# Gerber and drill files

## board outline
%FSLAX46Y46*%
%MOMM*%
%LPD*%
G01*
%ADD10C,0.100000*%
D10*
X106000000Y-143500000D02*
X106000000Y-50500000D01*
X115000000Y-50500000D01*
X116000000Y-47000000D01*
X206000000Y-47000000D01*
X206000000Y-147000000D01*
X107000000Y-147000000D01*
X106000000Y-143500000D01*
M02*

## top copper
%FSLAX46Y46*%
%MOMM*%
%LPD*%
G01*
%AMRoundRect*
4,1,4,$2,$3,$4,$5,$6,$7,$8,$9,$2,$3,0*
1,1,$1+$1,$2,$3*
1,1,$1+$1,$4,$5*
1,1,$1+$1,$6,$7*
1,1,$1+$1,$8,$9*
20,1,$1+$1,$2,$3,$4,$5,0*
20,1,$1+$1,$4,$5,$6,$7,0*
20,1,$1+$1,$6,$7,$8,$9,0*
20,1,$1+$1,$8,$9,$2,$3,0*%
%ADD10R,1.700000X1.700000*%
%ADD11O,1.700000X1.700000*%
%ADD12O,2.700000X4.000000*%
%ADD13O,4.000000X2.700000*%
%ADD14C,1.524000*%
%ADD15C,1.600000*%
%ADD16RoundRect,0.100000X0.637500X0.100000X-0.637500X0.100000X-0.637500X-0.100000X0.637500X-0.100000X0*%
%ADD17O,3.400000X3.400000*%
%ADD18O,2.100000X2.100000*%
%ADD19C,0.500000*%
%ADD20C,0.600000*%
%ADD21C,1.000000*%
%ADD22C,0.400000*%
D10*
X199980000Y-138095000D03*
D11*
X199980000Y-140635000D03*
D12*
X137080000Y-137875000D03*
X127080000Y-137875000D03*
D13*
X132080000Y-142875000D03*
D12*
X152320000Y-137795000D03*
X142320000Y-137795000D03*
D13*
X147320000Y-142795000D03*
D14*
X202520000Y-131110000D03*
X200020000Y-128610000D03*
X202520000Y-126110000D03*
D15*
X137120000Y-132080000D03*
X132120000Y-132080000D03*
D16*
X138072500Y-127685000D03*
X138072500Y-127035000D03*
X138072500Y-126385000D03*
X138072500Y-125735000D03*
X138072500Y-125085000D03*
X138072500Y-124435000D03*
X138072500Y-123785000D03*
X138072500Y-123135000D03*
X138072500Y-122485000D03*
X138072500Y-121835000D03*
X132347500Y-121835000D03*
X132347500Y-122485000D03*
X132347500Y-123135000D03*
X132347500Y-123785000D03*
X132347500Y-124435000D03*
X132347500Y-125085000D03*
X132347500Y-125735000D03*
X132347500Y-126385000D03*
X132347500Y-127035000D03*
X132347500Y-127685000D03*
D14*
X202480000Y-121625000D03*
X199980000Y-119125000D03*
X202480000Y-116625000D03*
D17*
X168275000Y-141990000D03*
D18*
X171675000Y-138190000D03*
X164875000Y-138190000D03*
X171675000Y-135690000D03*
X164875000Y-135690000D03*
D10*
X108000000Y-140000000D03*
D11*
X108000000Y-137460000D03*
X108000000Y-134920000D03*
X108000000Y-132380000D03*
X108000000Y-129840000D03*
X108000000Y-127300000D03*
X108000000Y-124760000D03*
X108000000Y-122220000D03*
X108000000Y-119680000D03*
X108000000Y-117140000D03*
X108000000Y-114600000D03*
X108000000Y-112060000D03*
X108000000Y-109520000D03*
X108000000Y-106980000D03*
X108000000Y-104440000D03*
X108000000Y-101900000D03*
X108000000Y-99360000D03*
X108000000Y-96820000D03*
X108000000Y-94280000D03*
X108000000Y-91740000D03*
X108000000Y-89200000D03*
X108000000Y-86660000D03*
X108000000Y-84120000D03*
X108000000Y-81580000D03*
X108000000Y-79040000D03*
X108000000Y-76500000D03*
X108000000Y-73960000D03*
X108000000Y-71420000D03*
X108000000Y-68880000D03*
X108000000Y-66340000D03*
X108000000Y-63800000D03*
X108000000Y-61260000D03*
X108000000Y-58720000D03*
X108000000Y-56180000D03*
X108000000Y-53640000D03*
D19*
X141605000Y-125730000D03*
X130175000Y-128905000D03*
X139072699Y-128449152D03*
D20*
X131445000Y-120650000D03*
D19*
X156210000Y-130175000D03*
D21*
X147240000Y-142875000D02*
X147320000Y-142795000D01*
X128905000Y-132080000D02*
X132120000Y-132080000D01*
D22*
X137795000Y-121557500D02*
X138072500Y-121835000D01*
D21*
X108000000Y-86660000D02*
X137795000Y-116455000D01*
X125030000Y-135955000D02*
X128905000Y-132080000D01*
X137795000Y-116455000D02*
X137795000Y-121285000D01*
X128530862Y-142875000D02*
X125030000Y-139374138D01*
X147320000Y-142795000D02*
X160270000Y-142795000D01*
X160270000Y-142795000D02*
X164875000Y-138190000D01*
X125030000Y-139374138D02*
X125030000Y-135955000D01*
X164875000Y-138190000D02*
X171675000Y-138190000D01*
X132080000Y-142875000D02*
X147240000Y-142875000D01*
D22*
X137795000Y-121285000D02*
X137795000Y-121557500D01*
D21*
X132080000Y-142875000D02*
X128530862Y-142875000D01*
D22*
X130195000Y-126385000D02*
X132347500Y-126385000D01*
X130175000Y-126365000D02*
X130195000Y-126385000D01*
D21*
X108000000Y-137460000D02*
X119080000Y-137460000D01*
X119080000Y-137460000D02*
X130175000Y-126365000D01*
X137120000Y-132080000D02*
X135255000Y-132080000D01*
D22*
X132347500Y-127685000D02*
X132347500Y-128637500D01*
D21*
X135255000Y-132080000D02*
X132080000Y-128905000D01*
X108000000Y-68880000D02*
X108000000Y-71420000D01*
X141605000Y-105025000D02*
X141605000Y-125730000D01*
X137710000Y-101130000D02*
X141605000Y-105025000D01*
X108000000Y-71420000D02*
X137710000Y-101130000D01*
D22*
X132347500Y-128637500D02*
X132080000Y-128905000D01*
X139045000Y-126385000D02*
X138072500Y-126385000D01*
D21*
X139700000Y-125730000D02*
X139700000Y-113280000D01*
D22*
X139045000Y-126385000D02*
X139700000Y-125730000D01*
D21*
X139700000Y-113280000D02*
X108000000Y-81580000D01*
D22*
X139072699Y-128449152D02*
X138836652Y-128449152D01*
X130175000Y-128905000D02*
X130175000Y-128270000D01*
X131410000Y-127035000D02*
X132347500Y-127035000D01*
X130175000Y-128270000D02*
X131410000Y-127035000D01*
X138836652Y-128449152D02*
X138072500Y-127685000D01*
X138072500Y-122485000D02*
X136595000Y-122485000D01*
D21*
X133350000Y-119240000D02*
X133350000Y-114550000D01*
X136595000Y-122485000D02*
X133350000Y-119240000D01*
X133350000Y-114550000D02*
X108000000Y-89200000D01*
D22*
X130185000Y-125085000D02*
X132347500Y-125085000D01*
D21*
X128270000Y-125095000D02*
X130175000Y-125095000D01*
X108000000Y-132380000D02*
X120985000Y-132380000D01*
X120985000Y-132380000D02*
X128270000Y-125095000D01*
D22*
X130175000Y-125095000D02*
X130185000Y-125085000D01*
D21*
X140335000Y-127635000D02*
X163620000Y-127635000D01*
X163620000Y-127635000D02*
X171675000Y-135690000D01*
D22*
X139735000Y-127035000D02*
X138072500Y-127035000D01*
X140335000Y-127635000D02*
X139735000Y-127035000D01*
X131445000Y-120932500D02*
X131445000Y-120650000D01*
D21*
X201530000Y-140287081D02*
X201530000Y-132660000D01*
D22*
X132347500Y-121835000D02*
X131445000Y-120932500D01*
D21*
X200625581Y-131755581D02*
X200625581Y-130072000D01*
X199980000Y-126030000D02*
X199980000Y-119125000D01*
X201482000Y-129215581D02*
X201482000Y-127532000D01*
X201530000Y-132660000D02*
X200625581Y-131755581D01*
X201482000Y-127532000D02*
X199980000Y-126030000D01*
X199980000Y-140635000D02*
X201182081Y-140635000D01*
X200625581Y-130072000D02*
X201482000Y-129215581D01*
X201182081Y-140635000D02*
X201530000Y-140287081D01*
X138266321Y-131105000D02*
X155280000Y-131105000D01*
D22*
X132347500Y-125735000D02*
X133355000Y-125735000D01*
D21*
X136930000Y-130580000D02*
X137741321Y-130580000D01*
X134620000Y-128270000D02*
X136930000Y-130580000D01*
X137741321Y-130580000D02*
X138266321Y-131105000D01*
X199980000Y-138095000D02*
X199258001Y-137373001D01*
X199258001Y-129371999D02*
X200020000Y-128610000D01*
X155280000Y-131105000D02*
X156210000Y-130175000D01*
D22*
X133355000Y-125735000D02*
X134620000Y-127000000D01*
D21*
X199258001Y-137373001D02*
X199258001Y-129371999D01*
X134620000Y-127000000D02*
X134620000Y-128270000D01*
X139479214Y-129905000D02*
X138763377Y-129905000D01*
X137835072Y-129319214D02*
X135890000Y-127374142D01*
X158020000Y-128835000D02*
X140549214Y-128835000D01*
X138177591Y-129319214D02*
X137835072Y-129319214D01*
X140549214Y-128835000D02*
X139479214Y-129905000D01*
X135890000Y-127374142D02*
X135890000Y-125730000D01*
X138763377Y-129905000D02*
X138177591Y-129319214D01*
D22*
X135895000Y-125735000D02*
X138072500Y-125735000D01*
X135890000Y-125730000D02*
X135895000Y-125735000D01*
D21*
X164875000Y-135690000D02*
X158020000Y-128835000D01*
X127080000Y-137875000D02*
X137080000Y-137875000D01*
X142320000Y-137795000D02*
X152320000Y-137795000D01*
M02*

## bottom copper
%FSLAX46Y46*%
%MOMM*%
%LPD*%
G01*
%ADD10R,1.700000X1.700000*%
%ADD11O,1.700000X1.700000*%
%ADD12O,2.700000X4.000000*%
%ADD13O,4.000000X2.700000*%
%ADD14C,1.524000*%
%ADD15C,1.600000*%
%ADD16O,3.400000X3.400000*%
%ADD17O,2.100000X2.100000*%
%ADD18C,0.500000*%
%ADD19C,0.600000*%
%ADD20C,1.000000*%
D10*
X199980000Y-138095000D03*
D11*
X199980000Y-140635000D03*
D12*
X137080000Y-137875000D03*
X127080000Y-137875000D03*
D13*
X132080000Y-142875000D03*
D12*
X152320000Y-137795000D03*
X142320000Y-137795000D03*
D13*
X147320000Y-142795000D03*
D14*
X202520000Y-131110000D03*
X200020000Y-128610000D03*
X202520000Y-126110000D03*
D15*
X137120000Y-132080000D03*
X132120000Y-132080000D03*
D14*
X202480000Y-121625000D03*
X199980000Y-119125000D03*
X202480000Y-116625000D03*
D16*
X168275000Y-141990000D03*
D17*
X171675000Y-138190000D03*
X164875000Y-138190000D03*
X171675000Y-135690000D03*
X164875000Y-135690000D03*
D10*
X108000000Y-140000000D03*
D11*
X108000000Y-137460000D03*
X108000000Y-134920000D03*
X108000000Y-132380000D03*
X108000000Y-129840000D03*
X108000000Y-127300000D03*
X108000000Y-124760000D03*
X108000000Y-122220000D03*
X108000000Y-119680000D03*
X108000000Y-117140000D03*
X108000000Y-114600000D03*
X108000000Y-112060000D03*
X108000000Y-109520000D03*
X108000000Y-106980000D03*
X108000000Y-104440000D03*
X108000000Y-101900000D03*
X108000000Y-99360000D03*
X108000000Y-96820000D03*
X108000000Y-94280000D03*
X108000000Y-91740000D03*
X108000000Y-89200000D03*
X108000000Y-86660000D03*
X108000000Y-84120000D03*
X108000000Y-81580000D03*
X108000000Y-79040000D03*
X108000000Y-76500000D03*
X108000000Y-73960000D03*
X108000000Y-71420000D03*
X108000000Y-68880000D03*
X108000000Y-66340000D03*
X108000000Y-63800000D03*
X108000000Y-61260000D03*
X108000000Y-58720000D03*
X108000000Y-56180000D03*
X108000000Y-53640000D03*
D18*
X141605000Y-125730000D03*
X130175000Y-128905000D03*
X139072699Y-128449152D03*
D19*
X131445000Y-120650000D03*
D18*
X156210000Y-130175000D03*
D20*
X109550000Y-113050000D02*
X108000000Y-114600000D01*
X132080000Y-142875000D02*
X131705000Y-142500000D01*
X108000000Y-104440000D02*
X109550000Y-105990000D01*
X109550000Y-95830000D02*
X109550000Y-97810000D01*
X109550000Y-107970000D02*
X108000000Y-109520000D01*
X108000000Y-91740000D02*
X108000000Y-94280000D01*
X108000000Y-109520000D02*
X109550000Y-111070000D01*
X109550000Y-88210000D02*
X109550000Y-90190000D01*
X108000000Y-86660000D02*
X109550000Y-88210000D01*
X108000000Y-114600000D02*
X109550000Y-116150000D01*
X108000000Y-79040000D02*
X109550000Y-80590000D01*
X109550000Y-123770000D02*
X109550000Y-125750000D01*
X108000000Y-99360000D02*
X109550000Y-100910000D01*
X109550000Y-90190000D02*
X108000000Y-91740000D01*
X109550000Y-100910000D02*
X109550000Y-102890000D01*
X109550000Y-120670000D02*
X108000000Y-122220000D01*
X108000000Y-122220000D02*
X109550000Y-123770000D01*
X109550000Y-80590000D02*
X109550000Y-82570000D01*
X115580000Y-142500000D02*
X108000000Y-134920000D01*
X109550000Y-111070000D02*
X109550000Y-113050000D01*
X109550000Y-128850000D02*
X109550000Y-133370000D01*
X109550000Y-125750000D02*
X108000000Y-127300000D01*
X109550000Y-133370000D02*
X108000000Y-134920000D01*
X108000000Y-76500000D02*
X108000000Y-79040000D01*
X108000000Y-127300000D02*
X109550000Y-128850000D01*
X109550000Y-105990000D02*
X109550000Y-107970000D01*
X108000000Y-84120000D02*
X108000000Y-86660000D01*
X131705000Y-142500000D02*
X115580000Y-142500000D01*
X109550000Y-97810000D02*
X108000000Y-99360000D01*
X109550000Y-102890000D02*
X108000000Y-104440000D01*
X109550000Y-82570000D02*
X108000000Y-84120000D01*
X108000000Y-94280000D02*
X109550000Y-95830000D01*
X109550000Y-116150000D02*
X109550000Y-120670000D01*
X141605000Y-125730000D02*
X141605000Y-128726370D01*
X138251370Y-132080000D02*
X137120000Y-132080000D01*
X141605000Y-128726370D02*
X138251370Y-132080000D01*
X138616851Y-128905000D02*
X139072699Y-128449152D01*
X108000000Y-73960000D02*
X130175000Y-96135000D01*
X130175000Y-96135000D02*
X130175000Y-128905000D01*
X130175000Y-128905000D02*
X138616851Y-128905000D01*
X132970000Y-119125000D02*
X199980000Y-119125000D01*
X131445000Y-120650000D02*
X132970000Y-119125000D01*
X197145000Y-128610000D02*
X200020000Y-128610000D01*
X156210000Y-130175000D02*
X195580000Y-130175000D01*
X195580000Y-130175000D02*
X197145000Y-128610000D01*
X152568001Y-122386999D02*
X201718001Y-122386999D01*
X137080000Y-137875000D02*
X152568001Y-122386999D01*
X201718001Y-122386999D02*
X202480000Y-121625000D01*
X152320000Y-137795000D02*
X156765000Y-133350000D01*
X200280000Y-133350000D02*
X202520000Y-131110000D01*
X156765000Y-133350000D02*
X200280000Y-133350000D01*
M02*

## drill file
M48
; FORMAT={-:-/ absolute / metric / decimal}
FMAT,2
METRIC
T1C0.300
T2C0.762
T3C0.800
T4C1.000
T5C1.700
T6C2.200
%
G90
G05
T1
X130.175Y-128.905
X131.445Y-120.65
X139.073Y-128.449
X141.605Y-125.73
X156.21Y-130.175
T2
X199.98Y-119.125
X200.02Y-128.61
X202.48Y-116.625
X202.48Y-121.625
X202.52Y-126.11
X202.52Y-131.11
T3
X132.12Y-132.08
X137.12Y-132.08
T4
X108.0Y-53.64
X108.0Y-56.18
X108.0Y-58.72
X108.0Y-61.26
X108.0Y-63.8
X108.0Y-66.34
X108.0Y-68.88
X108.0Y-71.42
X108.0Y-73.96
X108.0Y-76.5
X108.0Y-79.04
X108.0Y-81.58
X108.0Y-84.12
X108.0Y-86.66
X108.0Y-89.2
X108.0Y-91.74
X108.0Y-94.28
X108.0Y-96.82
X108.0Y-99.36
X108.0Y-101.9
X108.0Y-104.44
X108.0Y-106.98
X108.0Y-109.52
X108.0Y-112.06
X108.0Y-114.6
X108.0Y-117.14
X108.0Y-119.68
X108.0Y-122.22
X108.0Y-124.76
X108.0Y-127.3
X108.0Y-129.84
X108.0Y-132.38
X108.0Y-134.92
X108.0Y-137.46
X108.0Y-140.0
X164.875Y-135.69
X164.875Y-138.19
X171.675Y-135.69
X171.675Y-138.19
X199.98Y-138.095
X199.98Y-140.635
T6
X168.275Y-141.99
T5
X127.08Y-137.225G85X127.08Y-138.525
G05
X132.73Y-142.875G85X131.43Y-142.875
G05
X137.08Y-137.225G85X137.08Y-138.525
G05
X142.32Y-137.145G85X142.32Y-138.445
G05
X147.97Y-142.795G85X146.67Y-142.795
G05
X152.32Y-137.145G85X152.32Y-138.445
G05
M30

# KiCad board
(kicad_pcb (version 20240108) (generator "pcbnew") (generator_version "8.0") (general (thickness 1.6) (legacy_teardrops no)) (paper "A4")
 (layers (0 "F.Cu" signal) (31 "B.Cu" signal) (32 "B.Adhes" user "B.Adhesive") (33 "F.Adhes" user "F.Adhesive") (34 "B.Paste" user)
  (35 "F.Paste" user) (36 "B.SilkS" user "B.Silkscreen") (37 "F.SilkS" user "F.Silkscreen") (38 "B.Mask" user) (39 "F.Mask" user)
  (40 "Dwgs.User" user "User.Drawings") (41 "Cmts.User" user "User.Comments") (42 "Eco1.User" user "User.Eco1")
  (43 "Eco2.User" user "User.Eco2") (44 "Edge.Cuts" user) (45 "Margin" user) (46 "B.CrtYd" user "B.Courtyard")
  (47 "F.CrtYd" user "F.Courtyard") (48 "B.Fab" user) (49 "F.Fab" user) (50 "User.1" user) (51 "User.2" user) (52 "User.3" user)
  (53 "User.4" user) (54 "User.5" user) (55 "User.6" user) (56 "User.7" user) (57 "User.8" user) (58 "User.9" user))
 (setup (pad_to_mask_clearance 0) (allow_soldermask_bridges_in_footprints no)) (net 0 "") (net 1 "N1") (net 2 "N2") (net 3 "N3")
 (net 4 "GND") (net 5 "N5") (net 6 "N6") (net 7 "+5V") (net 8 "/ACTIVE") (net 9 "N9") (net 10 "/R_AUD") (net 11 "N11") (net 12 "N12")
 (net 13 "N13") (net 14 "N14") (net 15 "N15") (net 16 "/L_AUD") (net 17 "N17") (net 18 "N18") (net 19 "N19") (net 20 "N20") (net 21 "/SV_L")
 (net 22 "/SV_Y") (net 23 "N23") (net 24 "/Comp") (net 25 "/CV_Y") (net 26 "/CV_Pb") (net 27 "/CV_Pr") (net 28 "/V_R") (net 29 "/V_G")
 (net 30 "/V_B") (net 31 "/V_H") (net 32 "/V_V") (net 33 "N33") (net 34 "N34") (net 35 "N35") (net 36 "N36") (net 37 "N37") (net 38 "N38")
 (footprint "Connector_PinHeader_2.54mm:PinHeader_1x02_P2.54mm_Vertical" (layer "F.Cu") (at 199.98 138.095)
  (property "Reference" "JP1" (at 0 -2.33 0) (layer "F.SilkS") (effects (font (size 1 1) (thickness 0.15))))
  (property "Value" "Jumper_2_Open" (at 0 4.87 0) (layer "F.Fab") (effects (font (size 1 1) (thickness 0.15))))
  (pad "1" thru_hole rect (at 0 0) (size 1.7 1.7) (drill 1) (layers "*.Cu" "*.Mask") (remove_unused_layers no) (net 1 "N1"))
  (pad "2" thru_hole oval (at 0 2.54) (size 1.7 1.7) (drill 1) (layers "*.Cu" "*.Mask") (remove_unused_layers no) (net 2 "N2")))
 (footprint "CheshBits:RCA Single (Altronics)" (layer "F.Cu") (at 132.08 137.875 180)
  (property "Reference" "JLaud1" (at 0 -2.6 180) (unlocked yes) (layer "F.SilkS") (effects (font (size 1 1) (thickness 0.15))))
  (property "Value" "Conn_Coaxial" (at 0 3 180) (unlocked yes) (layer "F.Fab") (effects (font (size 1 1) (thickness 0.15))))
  (pad "1" thru_hole oval (at -5 0 270) (size 4 2.7) (drill oval 3 1.7) (layers "*.Cu" "*.Mask") (remove_unused_layers no) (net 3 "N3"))
  (pad "1" thru_hole oval (at 5 0 270) (size 4 2.7) (drill oval 3 1.7) (layers "*.Cu" "*.Mask") (remove_unused_layers no) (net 3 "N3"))
  (pad "2" thru_hole oval (at 0 -5 180) (size 4 2.7) (drill oval 3 1.7) (layers "*.Cu" "*.Mask") (remove_unused_layers no) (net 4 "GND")))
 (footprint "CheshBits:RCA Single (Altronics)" (layer "F.Cu") (at 147.32 137.795 180)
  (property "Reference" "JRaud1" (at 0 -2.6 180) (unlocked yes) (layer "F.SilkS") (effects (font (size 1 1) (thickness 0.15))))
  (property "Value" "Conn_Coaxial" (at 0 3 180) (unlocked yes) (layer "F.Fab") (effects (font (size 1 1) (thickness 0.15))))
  (pad "1" thru_hole oval (at -5 0 270) (size 4 2.7) (drill oval 3 1.7) (layers "*.Cu" "*.Mask") (remove_unused_layers no) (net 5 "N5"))
  (pad "1" thru_hole oval (at 5 0 270) (size 4 2.7) (drill oval 3 1.7) (layers "*.Cu" "*.Mask") (remove_unused_layers no) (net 5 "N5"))
  (pad "2" thru_hole oval (at 0 -5 180) (size 4 2.7) (drill oval 3 1.7) (layers "*.Cu" "*.Mask") (remove_unused_layers no) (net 4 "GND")))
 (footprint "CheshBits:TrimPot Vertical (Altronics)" (layer "F.Cu") (at 193.62 128.61 90)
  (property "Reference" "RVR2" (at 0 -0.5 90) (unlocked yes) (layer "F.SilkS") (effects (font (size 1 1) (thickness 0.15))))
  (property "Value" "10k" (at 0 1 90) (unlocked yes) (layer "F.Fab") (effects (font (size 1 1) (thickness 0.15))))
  (pad "1" thru_hole circle (at -2.5 8.9 90) (size 1.524 1.524) (drill 0.762) (layers "*.Cu" "*.Mask") (remove_unused_layers no)
   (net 5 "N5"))
  (pad "2" thru_hole circle (at 0 6.4 90) (size 1.524 1.524) (drill 0.762) (layers "*.Cu" "*.Mask") (remove_unused_layers no) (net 1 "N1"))
  (pad "3" thru_hole circle (at 2.5 8.9 90) (size 1.524 1.524) (drill 0.762) (layers "*.Cu" "*.Mask") (remove_unused_layers no) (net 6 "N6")))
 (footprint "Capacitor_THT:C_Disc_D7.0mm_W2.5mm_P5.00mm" (layer "F.Cu") (at 137.12 132.08 180)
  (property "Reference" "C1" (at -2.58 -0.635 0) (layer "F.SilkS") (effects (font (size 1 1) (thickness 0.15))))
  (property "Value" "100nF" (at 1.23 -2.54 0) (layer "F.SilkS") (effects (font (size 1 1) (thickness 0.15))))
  (pad "1" thru_hole circle (at 0 0 180) (size 1.6 1.6) (drill 0.8) (layers "*.Cu" "*.Mask") (remove_unused_layers no) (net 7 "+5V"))
  (pad "2" thru_hole circle (at 5 0 180) (size 1.6 1.6) (drill 0.8) (layers "*.Cu" "*.Mask") (remove_unused_layers no) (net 4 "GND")))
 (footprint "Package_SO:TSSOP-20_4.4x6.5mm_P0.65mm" (layer "F.Cu") (at 135.21 124.76 180)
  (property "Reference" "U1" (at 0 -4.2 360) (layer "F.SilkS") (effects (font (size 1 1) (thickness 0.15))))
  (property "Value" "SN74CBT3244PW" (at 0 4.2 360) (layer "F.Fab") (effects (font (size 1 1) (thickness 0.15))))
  (pad "1" smd roundrect (at -2.8625 -2.925 180) (size 1.475 0.4) (layers "F.Cu" "F.Paste" "F.Mask") (roundrect_rratio 0.25)
   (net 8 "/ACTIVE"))
  (pad "2" smd roundrect (at -2.8625 -2.275 180) (size 1.475 0.4) (layers "F.Cu" "F.Paste" "F.Mask") (roundrect_rratio 0.25) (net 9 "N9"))
  (pad "3" smd roundrect (at -2.8625 -1.625 180) (size 1.475 0.4) (layers "F.Cu" "F.Paste" "F.Mask") (roundrect_rratio 0.25)
   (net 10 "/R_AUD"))
  (pad "4" smd roundrect (at -2.8625 -0.975 180) (size 1.475 0.4) (layers "F.Cu" "F.Paste" "F.Mask") (roundrect_rratio 0.25) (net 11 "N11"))
  (pad "5" smd roundrect (at -2.8625 -0.325 180) (size 1.475 0.4) (layers "F.Cu" "F.Paste" "F.Mask") (roundrect_rratio 0.25) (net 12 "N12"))
  (pad "6" smd roundrect (at -2.8625 0.325 180) (size 1.475 0.4) (layers "F.Cu" "F.Paste" "F.Mask") (roundrect_rratio 0.25) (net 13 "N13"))
  (pad "7" smd roundrect (at -2.8625 0.975 180) (size 1.475 0.4) (layers "F.Cu" "F.Paste" "F.Mask") (roundrect_rratio 0.25) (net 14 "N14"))
  (pad "8" smd roundrect (at -2.8625 1.625 180) (size 1.475 0.4) (layers "F.Cu" "F.Paste" "F.Mask") (roundrect_rratio 0.25) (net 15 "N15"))
  (pad "9" smd roundrect (at -2.8625 2.275 180) (size 1.475 0.4) (layers "F.Cu" "F.Paste" "F.Mask") (roundrect_rratio 0.25)
   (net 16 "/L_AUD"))
  (pad "10" smd roundrect (at -2.8625 2.925 180) (size 1.475 0.4) (layers "F.Cu" "F.Paste" "F.Mask") (roundrect_rratio 0.25) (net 4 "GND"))
  (pad "11" smd roundrect (at 2.8625 2.925 180) (size 1.475 0.4) (layers "F.Cu" "F.Paste" "F.Mask") (roundrect_rratio 0.25) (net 2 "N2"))
  (pad "12" smd roundrect (at 2.8625 2.275 180) (size 1.475 0.4) (layers "F.Cu" "F.Paste" "F.Mask") (roundrect_rratio 0.25) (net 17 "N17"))
  (pad "13" smd roundrect (at 2.8625 1.625 180) (size 1.475 0.4) (layers "F.Cu" "F.Paste" "F.Mask") (roundrect_rratio 0.25) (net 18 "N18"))
  (pad "14" smd roundrect (at 2.8625 0.975 180) (size 1.475 0.4) (layers "F.Cu" "F.Paste" "F.Mask") (roundrect_rratio 0.25) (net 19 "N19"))
  (pad "15" smd roundrect (at 2.8625 0.325 180) (size 1.475 0.4) (layers "F.Cu" "F.Paste" "F.Mask") (roundrect_rratio 0.25) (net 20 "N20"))
  (pad "16" smd roundrect (at 2.8625 -0.325 180) (size 1.475 0.4) (layers "F.Cu" "F.Paste" "F.Mask") (roundrect_rratio 0.25)
   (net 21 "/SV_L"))
  (pad "17" smd roundrect (at 2.8625 -0.975 180) (size 1.475 0.4) (layers "F.Cu" "F.Paste" "F.Mask") (roundrect_rratio 0.25) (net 1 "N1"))
  (pad "18" smd roundrect (at 2.8625 -1.625 180) (size 1.475 0.4) (layers "F.Cu" "F.Paste" "F.Mask") (roundrect_rratio 0.25)
   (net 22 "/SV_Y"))
  (pad "19" smd roundrect (at 2.8625 -2.275 180) (size 1.475 0.4) (layers "F.Cu" "F.Paste" "F.Mask") (roundrect_rratio 0.25)
   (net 8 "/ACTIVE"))
  (pad "20" smd roundrect (at 2.8625 -2.925 180) (size 1.475 0.4) (layers "F.Cu" "F.Paste" "F.Mask") (roundrect_rratio 0.25) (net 7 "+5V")))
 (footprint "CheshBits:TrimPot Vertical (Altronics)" (layer "F.Cu") (at 193.58 119.125 90)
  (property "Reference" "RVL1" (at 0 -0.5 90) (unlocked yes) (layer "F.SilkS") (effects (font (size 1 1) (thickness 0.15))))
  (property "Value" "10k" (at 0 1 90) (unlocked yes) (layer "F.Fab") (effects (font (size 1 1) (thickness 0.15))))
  (pad "1" thru_hole circle (at -2.5 8.9 90) (size 1.524 1.524) (drill 0.762) (layers "*.Cu" "*.Mask") (remove_unused_layers no)
   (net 3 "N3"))
  (pad "2" thru_hole circle (at 0 6.4 90) (size 1.524 1.524) (drill 0.762) (layers "*.Cu" "*.Mask") (remove_unused_layers no) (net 2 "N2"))
  (pad "3" thru_hole circle (at 2.5 8.9 90) (size 1.524 1.524) (drill 0.762) (layers "*.Cu" "*.Mask") (remove_unused_layers no)
   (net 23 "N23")))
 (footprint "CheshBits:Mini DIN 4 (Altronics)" (layer "F.Cu") (at 168.275 148.59 180)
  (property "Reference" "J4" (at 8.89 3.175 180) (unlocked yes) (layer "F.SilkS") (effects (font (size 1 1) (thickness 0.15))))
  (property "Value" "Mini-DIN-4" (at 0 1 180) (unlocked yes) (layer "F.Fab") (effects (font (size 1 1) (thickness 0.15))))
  (pad "" thru_hole oval (at 0 6.6 270) (size 3.4 3.4) (drill oval 2.2) (layers "*.Cu" "*.Mask") (remove_unused_layers no))
  (pad "1" thru_hole oval (at -3.4 10.4 270) (size 2.1 2.1) (drill oval 1) (layers "*.Cu" "*.Mask") (remove_unused_layers no) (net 4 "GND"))
  (pad "2" thru_hole oval (at 3.4 10.4 270) (size 2.1 2.1) (drill oval 1) (layers "*.Cu" "*.Mask") (remove_unused_layers no) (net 4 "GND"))
  (pad "3" thru_hole oval (at -3.4 12.9 270) (size 2.1 2.1) (drill oval 1) (layers "*.Cu" "*.Mask") (remove_unused_layers no) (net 9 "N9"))
  (pad "4" thru_hole oval (at 3.4 12.9 270) (size 2.1 2.1) (drill oval 1) (layers "*.Cu" "*.Mask") (remove_unused_layers no) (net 11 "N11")))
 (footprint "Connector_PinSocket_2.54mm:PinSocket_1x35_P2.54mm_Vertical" (layer "B.Cu") (at 108 140)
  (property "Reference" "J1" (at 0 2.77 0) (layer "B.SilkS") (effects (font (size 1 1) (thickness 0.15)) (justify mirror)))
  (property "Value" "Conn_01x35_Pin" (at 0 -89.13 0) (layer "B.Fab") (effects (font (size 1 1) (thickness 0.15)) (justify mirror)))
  (pad "1" thru_hole rect (at 0 0) (size 1.7 1.7) (drill 1) (layers "*.Cu" "*.Mask") (remove_unused_layers no) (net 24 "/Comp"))
  (pad "2" thru_hole oval (at 0 -2.54) (size 1.7 1.7) (drill 1) (layers "*.Cu" "*.Mask") (remove_unused_layers no) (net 22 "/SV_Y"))
  (pad "3" thru_hole oval (at 0 -5.08) (size 1.7 1.7) (drill 1) (layers "*.Cu" "*.Mask") (remove_unused_layers no) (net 4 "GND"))
  (pad "4" thru_hole oval (at 0 -7.62) (size 1.7 1.7) (drill 1) (layers "*.Cu" "*.Mask") (remove_unused_layers no) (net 21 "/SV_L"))
  (pad "5" thru_hole oval (at 0 -10.16) (size 1.7 1.7) (drill 1) (layers "*.Cu" "*.Mask") (remove_unused_layers no) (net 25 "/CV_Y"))
  (pad "6" thru_hole oval (at 0 -12.7) (size 1.7 1.7) (drill 1) (layers "*.Cu" "*.Mask") (remove_unused_layers no) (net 4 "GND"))
  (pad "7" thru_hole oval (at 0 -15.24) (size 1.7 1.7) (drill 1) (layers "*.Cu" "*.Mask") (remove_unused_layers no) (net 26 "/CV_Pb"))
  (pad "8" thru_hole oval (at 0 -17.78) (size 1.7 1.7) (drill 1) (layers "*.Cu" "*.Mask") (remove_unused_layers no) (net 4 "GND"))
  (pad "9" thru_hole oval (at 0 -20.32) (size 1.7 1.7) (drill 1) (layers "*.Cu" "*.Mask") (remove_unused_layers no) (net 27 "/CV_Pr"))
  (pad "10" thru_hole oval (at 0 -22.86) (size 1.7 1.7) (drill 1) (layers "*.Cu" "*.Mask") (remove_unused_layers no) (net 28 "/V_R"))
  (pad "11" thru_hole oval (at 0 -25.4) (size 1.7 1.7) (drill 1) (layers "*.Cu" "*.Mask") (remove_unused_layers no) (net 4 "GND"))
  (pad "12" thru_hole oval (at 0 -27.94) (size 1.7 1.7) (drill 1) (layers "*.Cu" "*.Mask") (remove_unused_layers no) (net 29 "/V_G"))
  (pad "13" thru_hole oval (at 0 -30.48) (size 1.7 1.7) (drill 1) (layers "*.Cu" "*.Mask") (remove_unused_layers no) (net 4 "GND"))
  (pad "14" thru_hole oval (at 0 -33.02) (size 1.7 1.7) (drill 1) (layers "*.Cu" "*.Mask") (remove_unused_layers no) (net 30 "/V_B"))
  (pad "15" thru_hole oval (at 0 -35.56) (size 1.7 1.7) (drill 1) (layers "*.Cu" "*.Mask") (remove_unused_layers no) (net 4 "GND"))
  (pad "16" thru_hole oval (at 0 -38.1) (size 1.7 1.7) (drill 1) (layers "*.Cu" "*.Mask") (remove_unused_layers no) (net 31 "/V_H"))
  (pad "17" thru_hole oval (at 0 -40.64) (size 1.7 1.7) (drill 1) (layers "*.Cu" "*.Mask") (remove_unused_layers no) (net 4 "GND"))
  (pad "18" thru_hole oval (at 0 -43.18) (size 1.7 1.7) (drill 1) (layers "*.Cu" "*.Mask") (remove_unused_layers no) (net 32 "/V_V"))
  (pad "19" thru_hole oval (at 0 -45.72) (size 1.7 1.7) (drill 1) (layers "*.Cu" "*.Mask") (remove_unused_layers no) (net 4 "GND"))
  (pad "20" thru_hole oval (at 0 -48.26) (size 1.7 1.7) (drill 1) (layers "*.Cu" "*.Mask") (remove_unused_layers no) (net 4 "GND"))
  (pad "21" thru_hole oval (at 0 -50.8) (size 1.7 1.7) (drill 1) (layers "*.Cu" "*.Mask") (remove_unused_layers no) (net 16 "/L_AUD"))
  (pad "22" thru_hole oval (at 0 -53.34) (size 1.7 1.7) (drill 1) (layers "*.Cu" "*.Mask") (remove_unused_layers no) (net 4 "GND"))
  (pad "23" thru_hole oval (at 0 -55.88) (size 1.7 1.7) (drill 1) (layers "*.Cu" "*.Mask") (remove_unused_layers no) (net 4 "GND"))
  (pad "24" thru_hole oval (at 0 -58.42) (size 1.7 1.7) (drill 1) (layers "*.Cu" "*.Mask") (remove_unused_layers no) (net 10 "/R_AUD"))
  (pad "25" thru_hole oval (at 0 -60.96) (size 1.7 1.7) (drill 1) (layers "*.Cu" "*.Mask") (remove_unused_layers no) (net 4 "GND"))
  (pad "26" thru_hole oval (at 0 -63.5) (size 1.7 1.7) (drill 1) (layers "*.Cu" "*.Mask") (remove_unused_layers no) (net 4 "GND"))
  (pad "27" thru_hole oval (at 0 -66.04) (size 1.7 1.7) (drill 1) (layers "*.Cu" "*.Mask") (remove_unused_layers no) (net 8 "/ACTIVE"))
  (pad "28" thru_hole oval (at 0 -68.58) (size 1.7 1.7) (drill 1) (layers "*.Cu" "*.Mask") (remove_unused_layers no) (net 7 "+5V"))
  (pad "29" thru_hole oval (at 0 -71.12) (size 1.7 1.7) (drill 1) (layers "*.Cu" "*.Mask") (remove_unused_layers no) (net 7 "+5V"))
  (pad "30" thru_hole oval (at 0 -73.66) (size 1.7 1.7) (drill 1) (layers "*.Cu" "*.Mask") (remove_unused_layers no) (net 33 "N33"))
  (pad "31" thru_hole oval (at 0 -76.2) (size 1.7 1.7) (drill 1) (layers "*.Cu" "*.Mask") (remove_unused_layers no) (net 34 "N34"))
  (pad "32" thru_hole oval (at 0 -78.74) (size 1.7 1.7) (drill 1) (layers "*.Cu" "*.Mask") (remove_unused_layers no) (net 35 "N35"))
  (pad "33" thru_hole oval (at 0 -81.28) (size 1.7 1.7) (drill 1) (layers "*.Cu" "*.Mask") (remove_unused_layers no) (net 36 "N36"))
  (pad "34" thru_hole oval (at 0 -83.82) (size 1.7 1.7) (drill 1) (layers "*.Cu" "*.Mask") (remove_unused_layers no) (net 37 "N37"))
  (pad "35" thru_hole oval (at 0 -86.36) (size 1.7 1.7) (drill 1) (layers "*.Cu" "*.Mask") (remove_unused_layers no) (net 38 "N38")))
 (gr_poly
  (pts (xy 106 143.5) (xy 106 50.5) (xy 115 50.5) (xy 116 47) (xy 206 47) (xy 206 147) (xy 107 147)) (stroke (width 0.1) (type solid))
  (fill none) (layer "Edge.Cuts"))
 (segment (start 147.24 142.875) (end 147.32 142.795) (width 1) (layer "F.Cu") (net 4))
 (segment (start 128.905 132.08) (end 132.12 132.08) (width 1) (layer "F.Cu") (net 4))
 (segment (start 137.795 121.5575) (end 138.0725 121.835) (width 0.4) (layer "F.Cu") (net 4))
 (segment (start 108 86.66) (end 137.795 116.455) (width 1) (layer "F.Cu") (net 4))
 (segment (start 125.03 135.955) (end 128.905 132.08) (width 1) (layer "F.Cu") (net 4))
 (segment (start 137.795 116.455) (end 137.795 121.285) (width 1) (layer "F.Cu") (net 4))
 (segment (start 128.530862 142.875) (end 125.03 139.374138) (width 1) (layer "F.Cu") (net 4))
 (segment (start 147.32 142.795) (end 160.27 142.795) (width 1) (layer "F.Cu") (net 4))
 (segment (start 160.27 142.795) (end 164.875 138.19) (width 1) (layer "F.Cu") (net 4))
 (segment (start 125.03 139.374138) (end 125.03 135.955) (width 1) (layer "F.Cu") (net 4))
 (segment (start 164.875 138.19) (end 171.675 138.19) (width 1) (layer "F.Cu") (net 4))
 (segment (start 132.08 142.875) (end 147.24 142.875) (width 1) (layer "F.Cu") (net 4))
 (segment (start 137.795 121.285) (end 137.795 121.5575) (width 0.4) (layer "F.Cu") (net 4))
 (segment (start 132.08 142.875) (end 128.530862 142.875) (width 1) (layer "F.Cu") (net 4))
 (segment (start 109.55 113.05) (end 108 114.6) (width 1) (layer "B.Cu") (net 4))
 (segment (start 132.08 142.875) (end 131.705 142.5) (width 1) (layer "B.Cu") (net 4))
 (segment (start 108 104.44) (end 109.55 105.99) (width 1) (layer "B.Cu") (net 4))
 (segment (start 109.55 95.83) (end 109.55 97.81) (width 1) (layer "B.Cu") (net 4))
 (segment (start 109.55 107.97) (end 108 109.52) (width 1) (layer "B.Cu") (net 4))
 (segment (start 108 91.74) (end 108 94.28) (width 1) (layer "B.Cu") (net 4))
 (segment (start 108 109.52) (end 109.55 111.07) (width 1) (layer "B.Cu") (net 4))
 (segment (start 109.55 88.21) (end 109.55 90.19) (width 1) (layer "B.Cu") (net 4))
 (segment (start 108 86.66) (end 109.55 88.21) (width 1) (layer "B.Cu") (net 4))
 (segment (start 108 114.6) (end 109.55 116.15) (width 1) (layer "B.Cu") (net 4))
 (segment (start 108 79.04) (end 109.55 80.59) (width 1) (layer "B.Cu") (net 4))
 (segment (start 109.55 123.77) (end 109.55 125.75) (width 1) (layer "B.Cu") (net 4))
 (segment (start 108 99.36) (end 109.55 100.91) (width 1) (layer "B.Cu") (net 4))
 (segment (start 109.55 90.19) (end 108 91.74) (width 1) (layer "B.Cu") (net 4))
 (segment (start 109.55 100.91) (end 109.55 102.89) (width 1) (layer "B.Cu") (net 4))
 (segment (start 109.55 120.67) (end 108 122.22) (width 1) (layer "B.Cu") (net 4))
 (segment (start 108 122.22) (end 109.55 123.77) (width 1) (layer "B.Cu") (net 4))
 (segment (start 109.55 80.59) (end 109.55 82.57) (width 1) (layer "B.Cu") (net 4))
 (segment (start 115.58 142.5) (end 108 134.92) (width 1) (layer "B.Cu") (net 4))
 (segment (start 109.55 111.07) (end 109.55 113.05) (width 1) (layer "B.Cu") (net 4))
 (segment (start 109.55 128.85) (end 109.55 133.37) (width 1) (layer "B.Cu") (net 4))
 (segment (start 109.55 125.75) (end 108 127.3) (width 1) (layer "B.Cu") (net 4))
 (segment (start 109.55 133.37) (end 108 134.92) (width 1) (layer "B.Cu") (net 4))
 (segment (start 108 76.5) (end 108 79.04) (width 1) (layer "B.Cu") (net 4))
 (segment (start 108 127.3) (end 109.55 128.85) (width 1) (layer "B.Cu") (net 4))
 (segment (start 109.55 105.99) (end 109.55 107.97) (width 1) (layer "B.Cu") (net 4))
 (segment (start 108 84.12) (end 108 86.66) (width 1) (layer "B.Cu") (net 4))
 (segment (start 131.705 142.5) (end 115.58 142.5) (width 1) (layer "B.Cu") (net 4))
 (segment (start 109.55 97.81) (end 108 99.36) (width 1) (layer "B.Cu") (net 4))
 (segment (start 109.55 102.89) (end 108 104.44) (width 1) (layer "B.Cu") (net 4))
 (segment (start 109.55 82.57) (end 108 84.12) (width 1) (layer "B.Cu") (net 4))
 (segment (start 108 94.28) (end 109.55 95.83) (width 1) (layer "B.Cu") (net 4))
 (segment (start 109.55 116.15) (end 109.55 120.67) (width 1) (layer "B.Cu") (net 4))
 (segment (start 130.195 126.385) (end 132.3475 126.385) (width 0.4) (layer "F.Cu") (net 22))
 (segment (start 130.175 126.365) (end 130.195 126.385) (width 0.4) (layer "F.Cu") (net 22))
 (segment (start 108 137.46) (end 119.08 137.46) (width 1) (layer "F.Cu") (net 22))
 (segment (start 119.08 137.46) (end 130.175 126.365) (width 1) (layer "F.Cu") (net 22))
 (segment (start 137.12 132.08) (end 135.255 132.08) (width 1) (layer "F.Cu") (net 7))
 (segment (start 132.3475 127.685) (end 132.3475 128.6375) (width 0.4) (layer "F.Cu") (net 7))
 (segment (start 135.255 132.08) (end 132.08 128.905) (width 1) (layer "F.Cu") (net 7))
 (segment (start 108 68.88) (end 108 71.42) (width 1) (layer "F.Cu") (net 7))
 (segment (start 141.605 105.025) (end 141.605 125.73) (width 1) (layer "F.Cu") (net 7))
 (segment (start 137.71 101.13) (end 141.605 105.025) (width 1) (layer "F.Cu") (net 7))
 (segment (start 108 71.42) (end 137.71 101.13) (width 1) (layer "F.Cu") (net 7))
 (segment (start 132.3475 128.6375) (end 132.08 128.905) (width 0.4) (layer "F.Cu") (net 7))
 (via (at 141.605 125.73) (size 0.5) (drill 0.3) (layers "F.Cu" "B.Cu") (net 7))
 (segment (start 141.605 125.73) (end 141.605 128.72637) (width 1) (layer "B.Cu") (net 7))
 (segment (start 138.25137 132.08) (end 137.12 132.08) (width 1) (layer "B.Cu") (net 7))
 (segment (start 141.605 128.72637) (end 138.25137 132.08) (width 1) (layer "B.Cu") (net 7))
 (segment (start 139.045 126.385) (end 138.0725 126.385) (width 0.4) (layer "F.Cu") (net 10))
 (segment (start 139.7 125.73) (end 139.7 113.28) (width 1) (layer "F.Cu") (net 10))
 (segment (start 139.045 126.385) (end 139.7 125.73) (width 0.4) (layer "F.Cu") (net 10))
 (segment (start 139.7 113.28) (end 108 81.58) (width 1) (layer "F.Cu") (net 10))
 (segment (start 139.072699 128.449152) (end 138.836652 128.449152) (width 0.4) (layer "F.Cu") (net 8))
 (segment (start 130.175 128.905) (end 130.175 128.27) (width 0.4) (layer "F.Cu") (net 8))
 (segment (start 131.41 127.035) (end 132.3475 127.035) (width 0.4) (layer "F.Cu") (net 8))
 (segment (start 130.175 128.27) (end 131.41 127.035) (width 0.4) (layer "F.Cu") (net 8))
 (segment (start 138.836652 128.449152) (end 138.0725 127.685) (width 0.4) (layer "F.Cu") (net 8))
 (via (at 130.175 128.905) (size 0.5) (drill 0.3) (layers "F.Cu" "B.Cu") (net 8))
 (via (at 139.072699 128.449152) (size 0.5) (drill 0.3) (layers "F.Cu" "B.Cu") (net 8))
 (segment (start 138.616851 128.905) (end 139.072699 128.449152) (width 1) (layer "B.Cu") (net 8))
 (segment (start 108 73.96) (end 130.175 96.135) (width 1) (layer "B.Cu") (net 8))
 (segment (start 130.175 96.135) (end 130.175 128.905) (width 1) (layer "B.Cu") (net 8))
 (segment (start 130.175 128.905) (end 138.616851 128.905) (width 1) (layer "B.Cu") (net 8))
 (segment (start 138.0725 122.485) (end 136.595 122.485) (width 0.4) (layer "F.Cu") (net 16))
 (segment (start 133.35 119.24) (end 133.35 114.55) (width 1) (layer "F.Cu") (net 16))
 (segment (start 136.595 122.485) (end 133.35 119.24) (width 1) (layer "F.Cu") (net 16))
 (segment (start 133.35 114.55) (end 108 89.2) (width 1) (layer "F.Cu") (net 16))
 (segment (start 130.185 125.085) (end 132.3475 125.085) (width 0.4) (layer "F.Cu") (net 21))
 (segment (start 128.27 125.095) (end 130.175 125.095) (width 1) (layer "F.Cu") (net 21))
 (segment (start 108 132.38) (end 120.985 132.38) (width 1) (layer "F.Cu") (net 21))
 (segment (start 120.985 132.38) (end 128.27 125.095) (width 1) (layer "F.Cu") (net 21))
 (segment (start 130.175 125.095) (end 130.185 125.085) (width 0.4) (layer "F.Cu") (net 21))
 (segment (start 140.335 127.635) (end 163.62 127.635) (width 1) (layer "F.Cu") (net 9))
 (segment (start 163.62 127.635) (end 171.675 135.69) (width 1) (layer "F.Cu") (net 9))
 (segment (start 139.735 127.035) (end 138.0725 127.035) (width 0.4) (layer "F.Cu") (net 9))
 (segment (start 140.335 127.635) (end 139.735 127.035) (width 0.4) (layer "F.Cu") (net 9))
 (segment (start 131.445 120.9325) (end 131.445 120.65) (width 0.4) (layer "F.Cu") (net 2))
 (segment (start 201.53 140.287081) (end 201.53 132.66) (width 1) (layer "F.Cu") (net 2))
 (segment (start 132.3475 121.835) (end 131.445 120.9325) (width 0.4) (layer "F.Cu") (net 2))
 (segment (start 200.625581 131.755581) (end 200.625581 130.072) (width 1) (layer "F.Cu") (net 2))
 (segment (start 199.98 126.03) (end 199.98 119.125) (width 1) (layer "F.Cu") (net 2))
 (segment (start 201.482 129.215581) (end 201.482 127.532) (width 1) (layer "F.Cu") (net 2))
 (segment (start 201.53 132.66) (end 200.625581 131.755581) (width 1) (layer "F.Cu") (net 2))
 (segment (start 201.482 127.532) (end 199.98 126.03) (width 1) (layer "F.Cu") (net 2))
 (segment (start 199.98 140.635) (end 201.182081 140.635) (width 1) (layer "F.Cu") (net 2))
 (segment (start 200.625581 130.072) (end 201.482 129.215581) (width 1) (layer "F.Cu") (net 2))
 (segment (start 201.182081 140.635) (end 201.53 140.287081) (width 1) (layer "F.Cu") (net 2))
 (via (at 131.445 120.65) (size 0.6) (drill 0.3) (layers "F.Cu" "B.Cu") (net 2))
 (segment (start 132.97 119.125) (end 199.98 119.125) (width 1) (layer "B.Cu") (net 2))
 (segment (start 131.445 120.65) (end 132.97 119.125) (width 1) (layer "B.Cu") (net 2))
 (segment (start 138.266321 131.105) (end 155.28 131.105) (width 1) (layer "F.Cu") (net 1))
 (segment (start 132.3475 125.735) (end 133.355 125.735) (width 0.4) (layer "F.Cu") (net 1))
 (segment (start 136.93 130.58) (end 137.741321 130.58) (width 1) (layer "F.Cu") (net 1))
 (segment (start 134.62 128.27) (end 136.93 130.58) (width 1) (layer "F.Cu") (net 1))
 (segment (start 137.741321 130.58) (end 138.266321 131.105) (width 1) (layer "F.Cu") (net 1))
 (segment (start 199.98 138.095) (end 199.258001 137.373001) (width 1) (layer "F.Cu") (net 1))
 (segment (start 199.258001 129.371999) (end 200.02 128.61) (width 1) (layer "F.Cu") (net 1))
 (segment (start 155.28 131.105) (end 156.21 130.175) (width 1) (layer "F.Cu") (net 1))
 (segment (start 133.355 125.735) (end 134.62 127) (width 0.4) (layer "F.Cu") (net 1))
 (segment (start 199.258001 137.373001) (end 199.258001 129.371999) (width 1) (layer "F.Cu") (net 1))
 (segment (start 134.62 127) (end 134.62 128.27) (width 1) (layer "F.Cu") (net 1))
 (via (at 156.21 130.175) (size 0.5) (drill 0.3) (layers "F.Cu" "B.Cu") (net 1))
 (segment (start 197.145 128.61) (end 200.02 128.61) (width 1) (layer "B.Cu") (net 1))
 (segment (start 156.21 130.175) (end 195.58 130.175) (width 1) (layer "B.Cu") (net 1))
 (segment (start 195.58 130.175) (end 197.145 128.61) (width 1) (layer "B.Cu") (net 1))
 (segment (start 139.479214 129.905) (end 138.763377 129.905) (width 1) (layer "F.Cu") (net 11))
 (segment (start 137.835072 129.319214) (end 135.89 127.374142) (width 1) (layer "F.Cu") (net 11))
 (segment (start 158.02 128.835) (end 140.549214 128.835) (width 1) (layer "F.Cu") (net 11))
 (segment (start 138.177591 129.319214) (end 137.835072 129.319214) (width 1) (layer "F.Cu") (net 11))
 (segment (start 140.549214 128.835) (end 139.479214 129.905) (width 1) (layer "F.Cu") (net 11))
 (segment (start 135.89 127.374142) (end 135.89 125.73) (width 1) (layer "F.Cu") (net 11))
 (segment (start 138.763377 129.905) (end 138.177591 129.319214) (width 1) (layer "F.Cu") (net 11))
 (segment (start 135.895 125.735) (end 138.0725 125.735) (width 0.4) (layer "F.Cu") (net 11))
 (segment (start 135.89 125.73) (end 135.895 125.735) (width 0.4) (layer "F.Cu") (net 11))
 (segment (start 164.875 135.69) (end 158.02 128.835) (width 1) (layer "F.Cu") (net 11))
 (segment (start 127.08 137.875) (end 137.08 137.875) (width 1) (layer "F.Cu") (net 3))
 (segment (start 152.568001 122.386999) (end 201.718001 122.386999) (width 1) (layer "B.Cu") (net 3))
 (segment (start 137.08 137.875) (end 152.568001 122.386999) (width 1) (layer "B.Cu") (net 3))
 (segment (start 201.718001 122.386999) (end 202.48 121.625) (width 1) (layer "B.Cu") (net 3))
 (segment (start 142.32 137.795) (end 152.32 137.795) (width 1) (layer "F.Cu") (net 5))
 (segment (start 152.32 137.795) (end 156.765 133.35) (width 1) (layer "B.Cu") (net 5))
 (segment (start 200.28 133.35) (end 202.52 131.11) (width 1) (layer "B.Cu") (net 5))
 (segment (start 156.765 133.35) (end 200.28 133.35) (width 1) (layer "B.Cu") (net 5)))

